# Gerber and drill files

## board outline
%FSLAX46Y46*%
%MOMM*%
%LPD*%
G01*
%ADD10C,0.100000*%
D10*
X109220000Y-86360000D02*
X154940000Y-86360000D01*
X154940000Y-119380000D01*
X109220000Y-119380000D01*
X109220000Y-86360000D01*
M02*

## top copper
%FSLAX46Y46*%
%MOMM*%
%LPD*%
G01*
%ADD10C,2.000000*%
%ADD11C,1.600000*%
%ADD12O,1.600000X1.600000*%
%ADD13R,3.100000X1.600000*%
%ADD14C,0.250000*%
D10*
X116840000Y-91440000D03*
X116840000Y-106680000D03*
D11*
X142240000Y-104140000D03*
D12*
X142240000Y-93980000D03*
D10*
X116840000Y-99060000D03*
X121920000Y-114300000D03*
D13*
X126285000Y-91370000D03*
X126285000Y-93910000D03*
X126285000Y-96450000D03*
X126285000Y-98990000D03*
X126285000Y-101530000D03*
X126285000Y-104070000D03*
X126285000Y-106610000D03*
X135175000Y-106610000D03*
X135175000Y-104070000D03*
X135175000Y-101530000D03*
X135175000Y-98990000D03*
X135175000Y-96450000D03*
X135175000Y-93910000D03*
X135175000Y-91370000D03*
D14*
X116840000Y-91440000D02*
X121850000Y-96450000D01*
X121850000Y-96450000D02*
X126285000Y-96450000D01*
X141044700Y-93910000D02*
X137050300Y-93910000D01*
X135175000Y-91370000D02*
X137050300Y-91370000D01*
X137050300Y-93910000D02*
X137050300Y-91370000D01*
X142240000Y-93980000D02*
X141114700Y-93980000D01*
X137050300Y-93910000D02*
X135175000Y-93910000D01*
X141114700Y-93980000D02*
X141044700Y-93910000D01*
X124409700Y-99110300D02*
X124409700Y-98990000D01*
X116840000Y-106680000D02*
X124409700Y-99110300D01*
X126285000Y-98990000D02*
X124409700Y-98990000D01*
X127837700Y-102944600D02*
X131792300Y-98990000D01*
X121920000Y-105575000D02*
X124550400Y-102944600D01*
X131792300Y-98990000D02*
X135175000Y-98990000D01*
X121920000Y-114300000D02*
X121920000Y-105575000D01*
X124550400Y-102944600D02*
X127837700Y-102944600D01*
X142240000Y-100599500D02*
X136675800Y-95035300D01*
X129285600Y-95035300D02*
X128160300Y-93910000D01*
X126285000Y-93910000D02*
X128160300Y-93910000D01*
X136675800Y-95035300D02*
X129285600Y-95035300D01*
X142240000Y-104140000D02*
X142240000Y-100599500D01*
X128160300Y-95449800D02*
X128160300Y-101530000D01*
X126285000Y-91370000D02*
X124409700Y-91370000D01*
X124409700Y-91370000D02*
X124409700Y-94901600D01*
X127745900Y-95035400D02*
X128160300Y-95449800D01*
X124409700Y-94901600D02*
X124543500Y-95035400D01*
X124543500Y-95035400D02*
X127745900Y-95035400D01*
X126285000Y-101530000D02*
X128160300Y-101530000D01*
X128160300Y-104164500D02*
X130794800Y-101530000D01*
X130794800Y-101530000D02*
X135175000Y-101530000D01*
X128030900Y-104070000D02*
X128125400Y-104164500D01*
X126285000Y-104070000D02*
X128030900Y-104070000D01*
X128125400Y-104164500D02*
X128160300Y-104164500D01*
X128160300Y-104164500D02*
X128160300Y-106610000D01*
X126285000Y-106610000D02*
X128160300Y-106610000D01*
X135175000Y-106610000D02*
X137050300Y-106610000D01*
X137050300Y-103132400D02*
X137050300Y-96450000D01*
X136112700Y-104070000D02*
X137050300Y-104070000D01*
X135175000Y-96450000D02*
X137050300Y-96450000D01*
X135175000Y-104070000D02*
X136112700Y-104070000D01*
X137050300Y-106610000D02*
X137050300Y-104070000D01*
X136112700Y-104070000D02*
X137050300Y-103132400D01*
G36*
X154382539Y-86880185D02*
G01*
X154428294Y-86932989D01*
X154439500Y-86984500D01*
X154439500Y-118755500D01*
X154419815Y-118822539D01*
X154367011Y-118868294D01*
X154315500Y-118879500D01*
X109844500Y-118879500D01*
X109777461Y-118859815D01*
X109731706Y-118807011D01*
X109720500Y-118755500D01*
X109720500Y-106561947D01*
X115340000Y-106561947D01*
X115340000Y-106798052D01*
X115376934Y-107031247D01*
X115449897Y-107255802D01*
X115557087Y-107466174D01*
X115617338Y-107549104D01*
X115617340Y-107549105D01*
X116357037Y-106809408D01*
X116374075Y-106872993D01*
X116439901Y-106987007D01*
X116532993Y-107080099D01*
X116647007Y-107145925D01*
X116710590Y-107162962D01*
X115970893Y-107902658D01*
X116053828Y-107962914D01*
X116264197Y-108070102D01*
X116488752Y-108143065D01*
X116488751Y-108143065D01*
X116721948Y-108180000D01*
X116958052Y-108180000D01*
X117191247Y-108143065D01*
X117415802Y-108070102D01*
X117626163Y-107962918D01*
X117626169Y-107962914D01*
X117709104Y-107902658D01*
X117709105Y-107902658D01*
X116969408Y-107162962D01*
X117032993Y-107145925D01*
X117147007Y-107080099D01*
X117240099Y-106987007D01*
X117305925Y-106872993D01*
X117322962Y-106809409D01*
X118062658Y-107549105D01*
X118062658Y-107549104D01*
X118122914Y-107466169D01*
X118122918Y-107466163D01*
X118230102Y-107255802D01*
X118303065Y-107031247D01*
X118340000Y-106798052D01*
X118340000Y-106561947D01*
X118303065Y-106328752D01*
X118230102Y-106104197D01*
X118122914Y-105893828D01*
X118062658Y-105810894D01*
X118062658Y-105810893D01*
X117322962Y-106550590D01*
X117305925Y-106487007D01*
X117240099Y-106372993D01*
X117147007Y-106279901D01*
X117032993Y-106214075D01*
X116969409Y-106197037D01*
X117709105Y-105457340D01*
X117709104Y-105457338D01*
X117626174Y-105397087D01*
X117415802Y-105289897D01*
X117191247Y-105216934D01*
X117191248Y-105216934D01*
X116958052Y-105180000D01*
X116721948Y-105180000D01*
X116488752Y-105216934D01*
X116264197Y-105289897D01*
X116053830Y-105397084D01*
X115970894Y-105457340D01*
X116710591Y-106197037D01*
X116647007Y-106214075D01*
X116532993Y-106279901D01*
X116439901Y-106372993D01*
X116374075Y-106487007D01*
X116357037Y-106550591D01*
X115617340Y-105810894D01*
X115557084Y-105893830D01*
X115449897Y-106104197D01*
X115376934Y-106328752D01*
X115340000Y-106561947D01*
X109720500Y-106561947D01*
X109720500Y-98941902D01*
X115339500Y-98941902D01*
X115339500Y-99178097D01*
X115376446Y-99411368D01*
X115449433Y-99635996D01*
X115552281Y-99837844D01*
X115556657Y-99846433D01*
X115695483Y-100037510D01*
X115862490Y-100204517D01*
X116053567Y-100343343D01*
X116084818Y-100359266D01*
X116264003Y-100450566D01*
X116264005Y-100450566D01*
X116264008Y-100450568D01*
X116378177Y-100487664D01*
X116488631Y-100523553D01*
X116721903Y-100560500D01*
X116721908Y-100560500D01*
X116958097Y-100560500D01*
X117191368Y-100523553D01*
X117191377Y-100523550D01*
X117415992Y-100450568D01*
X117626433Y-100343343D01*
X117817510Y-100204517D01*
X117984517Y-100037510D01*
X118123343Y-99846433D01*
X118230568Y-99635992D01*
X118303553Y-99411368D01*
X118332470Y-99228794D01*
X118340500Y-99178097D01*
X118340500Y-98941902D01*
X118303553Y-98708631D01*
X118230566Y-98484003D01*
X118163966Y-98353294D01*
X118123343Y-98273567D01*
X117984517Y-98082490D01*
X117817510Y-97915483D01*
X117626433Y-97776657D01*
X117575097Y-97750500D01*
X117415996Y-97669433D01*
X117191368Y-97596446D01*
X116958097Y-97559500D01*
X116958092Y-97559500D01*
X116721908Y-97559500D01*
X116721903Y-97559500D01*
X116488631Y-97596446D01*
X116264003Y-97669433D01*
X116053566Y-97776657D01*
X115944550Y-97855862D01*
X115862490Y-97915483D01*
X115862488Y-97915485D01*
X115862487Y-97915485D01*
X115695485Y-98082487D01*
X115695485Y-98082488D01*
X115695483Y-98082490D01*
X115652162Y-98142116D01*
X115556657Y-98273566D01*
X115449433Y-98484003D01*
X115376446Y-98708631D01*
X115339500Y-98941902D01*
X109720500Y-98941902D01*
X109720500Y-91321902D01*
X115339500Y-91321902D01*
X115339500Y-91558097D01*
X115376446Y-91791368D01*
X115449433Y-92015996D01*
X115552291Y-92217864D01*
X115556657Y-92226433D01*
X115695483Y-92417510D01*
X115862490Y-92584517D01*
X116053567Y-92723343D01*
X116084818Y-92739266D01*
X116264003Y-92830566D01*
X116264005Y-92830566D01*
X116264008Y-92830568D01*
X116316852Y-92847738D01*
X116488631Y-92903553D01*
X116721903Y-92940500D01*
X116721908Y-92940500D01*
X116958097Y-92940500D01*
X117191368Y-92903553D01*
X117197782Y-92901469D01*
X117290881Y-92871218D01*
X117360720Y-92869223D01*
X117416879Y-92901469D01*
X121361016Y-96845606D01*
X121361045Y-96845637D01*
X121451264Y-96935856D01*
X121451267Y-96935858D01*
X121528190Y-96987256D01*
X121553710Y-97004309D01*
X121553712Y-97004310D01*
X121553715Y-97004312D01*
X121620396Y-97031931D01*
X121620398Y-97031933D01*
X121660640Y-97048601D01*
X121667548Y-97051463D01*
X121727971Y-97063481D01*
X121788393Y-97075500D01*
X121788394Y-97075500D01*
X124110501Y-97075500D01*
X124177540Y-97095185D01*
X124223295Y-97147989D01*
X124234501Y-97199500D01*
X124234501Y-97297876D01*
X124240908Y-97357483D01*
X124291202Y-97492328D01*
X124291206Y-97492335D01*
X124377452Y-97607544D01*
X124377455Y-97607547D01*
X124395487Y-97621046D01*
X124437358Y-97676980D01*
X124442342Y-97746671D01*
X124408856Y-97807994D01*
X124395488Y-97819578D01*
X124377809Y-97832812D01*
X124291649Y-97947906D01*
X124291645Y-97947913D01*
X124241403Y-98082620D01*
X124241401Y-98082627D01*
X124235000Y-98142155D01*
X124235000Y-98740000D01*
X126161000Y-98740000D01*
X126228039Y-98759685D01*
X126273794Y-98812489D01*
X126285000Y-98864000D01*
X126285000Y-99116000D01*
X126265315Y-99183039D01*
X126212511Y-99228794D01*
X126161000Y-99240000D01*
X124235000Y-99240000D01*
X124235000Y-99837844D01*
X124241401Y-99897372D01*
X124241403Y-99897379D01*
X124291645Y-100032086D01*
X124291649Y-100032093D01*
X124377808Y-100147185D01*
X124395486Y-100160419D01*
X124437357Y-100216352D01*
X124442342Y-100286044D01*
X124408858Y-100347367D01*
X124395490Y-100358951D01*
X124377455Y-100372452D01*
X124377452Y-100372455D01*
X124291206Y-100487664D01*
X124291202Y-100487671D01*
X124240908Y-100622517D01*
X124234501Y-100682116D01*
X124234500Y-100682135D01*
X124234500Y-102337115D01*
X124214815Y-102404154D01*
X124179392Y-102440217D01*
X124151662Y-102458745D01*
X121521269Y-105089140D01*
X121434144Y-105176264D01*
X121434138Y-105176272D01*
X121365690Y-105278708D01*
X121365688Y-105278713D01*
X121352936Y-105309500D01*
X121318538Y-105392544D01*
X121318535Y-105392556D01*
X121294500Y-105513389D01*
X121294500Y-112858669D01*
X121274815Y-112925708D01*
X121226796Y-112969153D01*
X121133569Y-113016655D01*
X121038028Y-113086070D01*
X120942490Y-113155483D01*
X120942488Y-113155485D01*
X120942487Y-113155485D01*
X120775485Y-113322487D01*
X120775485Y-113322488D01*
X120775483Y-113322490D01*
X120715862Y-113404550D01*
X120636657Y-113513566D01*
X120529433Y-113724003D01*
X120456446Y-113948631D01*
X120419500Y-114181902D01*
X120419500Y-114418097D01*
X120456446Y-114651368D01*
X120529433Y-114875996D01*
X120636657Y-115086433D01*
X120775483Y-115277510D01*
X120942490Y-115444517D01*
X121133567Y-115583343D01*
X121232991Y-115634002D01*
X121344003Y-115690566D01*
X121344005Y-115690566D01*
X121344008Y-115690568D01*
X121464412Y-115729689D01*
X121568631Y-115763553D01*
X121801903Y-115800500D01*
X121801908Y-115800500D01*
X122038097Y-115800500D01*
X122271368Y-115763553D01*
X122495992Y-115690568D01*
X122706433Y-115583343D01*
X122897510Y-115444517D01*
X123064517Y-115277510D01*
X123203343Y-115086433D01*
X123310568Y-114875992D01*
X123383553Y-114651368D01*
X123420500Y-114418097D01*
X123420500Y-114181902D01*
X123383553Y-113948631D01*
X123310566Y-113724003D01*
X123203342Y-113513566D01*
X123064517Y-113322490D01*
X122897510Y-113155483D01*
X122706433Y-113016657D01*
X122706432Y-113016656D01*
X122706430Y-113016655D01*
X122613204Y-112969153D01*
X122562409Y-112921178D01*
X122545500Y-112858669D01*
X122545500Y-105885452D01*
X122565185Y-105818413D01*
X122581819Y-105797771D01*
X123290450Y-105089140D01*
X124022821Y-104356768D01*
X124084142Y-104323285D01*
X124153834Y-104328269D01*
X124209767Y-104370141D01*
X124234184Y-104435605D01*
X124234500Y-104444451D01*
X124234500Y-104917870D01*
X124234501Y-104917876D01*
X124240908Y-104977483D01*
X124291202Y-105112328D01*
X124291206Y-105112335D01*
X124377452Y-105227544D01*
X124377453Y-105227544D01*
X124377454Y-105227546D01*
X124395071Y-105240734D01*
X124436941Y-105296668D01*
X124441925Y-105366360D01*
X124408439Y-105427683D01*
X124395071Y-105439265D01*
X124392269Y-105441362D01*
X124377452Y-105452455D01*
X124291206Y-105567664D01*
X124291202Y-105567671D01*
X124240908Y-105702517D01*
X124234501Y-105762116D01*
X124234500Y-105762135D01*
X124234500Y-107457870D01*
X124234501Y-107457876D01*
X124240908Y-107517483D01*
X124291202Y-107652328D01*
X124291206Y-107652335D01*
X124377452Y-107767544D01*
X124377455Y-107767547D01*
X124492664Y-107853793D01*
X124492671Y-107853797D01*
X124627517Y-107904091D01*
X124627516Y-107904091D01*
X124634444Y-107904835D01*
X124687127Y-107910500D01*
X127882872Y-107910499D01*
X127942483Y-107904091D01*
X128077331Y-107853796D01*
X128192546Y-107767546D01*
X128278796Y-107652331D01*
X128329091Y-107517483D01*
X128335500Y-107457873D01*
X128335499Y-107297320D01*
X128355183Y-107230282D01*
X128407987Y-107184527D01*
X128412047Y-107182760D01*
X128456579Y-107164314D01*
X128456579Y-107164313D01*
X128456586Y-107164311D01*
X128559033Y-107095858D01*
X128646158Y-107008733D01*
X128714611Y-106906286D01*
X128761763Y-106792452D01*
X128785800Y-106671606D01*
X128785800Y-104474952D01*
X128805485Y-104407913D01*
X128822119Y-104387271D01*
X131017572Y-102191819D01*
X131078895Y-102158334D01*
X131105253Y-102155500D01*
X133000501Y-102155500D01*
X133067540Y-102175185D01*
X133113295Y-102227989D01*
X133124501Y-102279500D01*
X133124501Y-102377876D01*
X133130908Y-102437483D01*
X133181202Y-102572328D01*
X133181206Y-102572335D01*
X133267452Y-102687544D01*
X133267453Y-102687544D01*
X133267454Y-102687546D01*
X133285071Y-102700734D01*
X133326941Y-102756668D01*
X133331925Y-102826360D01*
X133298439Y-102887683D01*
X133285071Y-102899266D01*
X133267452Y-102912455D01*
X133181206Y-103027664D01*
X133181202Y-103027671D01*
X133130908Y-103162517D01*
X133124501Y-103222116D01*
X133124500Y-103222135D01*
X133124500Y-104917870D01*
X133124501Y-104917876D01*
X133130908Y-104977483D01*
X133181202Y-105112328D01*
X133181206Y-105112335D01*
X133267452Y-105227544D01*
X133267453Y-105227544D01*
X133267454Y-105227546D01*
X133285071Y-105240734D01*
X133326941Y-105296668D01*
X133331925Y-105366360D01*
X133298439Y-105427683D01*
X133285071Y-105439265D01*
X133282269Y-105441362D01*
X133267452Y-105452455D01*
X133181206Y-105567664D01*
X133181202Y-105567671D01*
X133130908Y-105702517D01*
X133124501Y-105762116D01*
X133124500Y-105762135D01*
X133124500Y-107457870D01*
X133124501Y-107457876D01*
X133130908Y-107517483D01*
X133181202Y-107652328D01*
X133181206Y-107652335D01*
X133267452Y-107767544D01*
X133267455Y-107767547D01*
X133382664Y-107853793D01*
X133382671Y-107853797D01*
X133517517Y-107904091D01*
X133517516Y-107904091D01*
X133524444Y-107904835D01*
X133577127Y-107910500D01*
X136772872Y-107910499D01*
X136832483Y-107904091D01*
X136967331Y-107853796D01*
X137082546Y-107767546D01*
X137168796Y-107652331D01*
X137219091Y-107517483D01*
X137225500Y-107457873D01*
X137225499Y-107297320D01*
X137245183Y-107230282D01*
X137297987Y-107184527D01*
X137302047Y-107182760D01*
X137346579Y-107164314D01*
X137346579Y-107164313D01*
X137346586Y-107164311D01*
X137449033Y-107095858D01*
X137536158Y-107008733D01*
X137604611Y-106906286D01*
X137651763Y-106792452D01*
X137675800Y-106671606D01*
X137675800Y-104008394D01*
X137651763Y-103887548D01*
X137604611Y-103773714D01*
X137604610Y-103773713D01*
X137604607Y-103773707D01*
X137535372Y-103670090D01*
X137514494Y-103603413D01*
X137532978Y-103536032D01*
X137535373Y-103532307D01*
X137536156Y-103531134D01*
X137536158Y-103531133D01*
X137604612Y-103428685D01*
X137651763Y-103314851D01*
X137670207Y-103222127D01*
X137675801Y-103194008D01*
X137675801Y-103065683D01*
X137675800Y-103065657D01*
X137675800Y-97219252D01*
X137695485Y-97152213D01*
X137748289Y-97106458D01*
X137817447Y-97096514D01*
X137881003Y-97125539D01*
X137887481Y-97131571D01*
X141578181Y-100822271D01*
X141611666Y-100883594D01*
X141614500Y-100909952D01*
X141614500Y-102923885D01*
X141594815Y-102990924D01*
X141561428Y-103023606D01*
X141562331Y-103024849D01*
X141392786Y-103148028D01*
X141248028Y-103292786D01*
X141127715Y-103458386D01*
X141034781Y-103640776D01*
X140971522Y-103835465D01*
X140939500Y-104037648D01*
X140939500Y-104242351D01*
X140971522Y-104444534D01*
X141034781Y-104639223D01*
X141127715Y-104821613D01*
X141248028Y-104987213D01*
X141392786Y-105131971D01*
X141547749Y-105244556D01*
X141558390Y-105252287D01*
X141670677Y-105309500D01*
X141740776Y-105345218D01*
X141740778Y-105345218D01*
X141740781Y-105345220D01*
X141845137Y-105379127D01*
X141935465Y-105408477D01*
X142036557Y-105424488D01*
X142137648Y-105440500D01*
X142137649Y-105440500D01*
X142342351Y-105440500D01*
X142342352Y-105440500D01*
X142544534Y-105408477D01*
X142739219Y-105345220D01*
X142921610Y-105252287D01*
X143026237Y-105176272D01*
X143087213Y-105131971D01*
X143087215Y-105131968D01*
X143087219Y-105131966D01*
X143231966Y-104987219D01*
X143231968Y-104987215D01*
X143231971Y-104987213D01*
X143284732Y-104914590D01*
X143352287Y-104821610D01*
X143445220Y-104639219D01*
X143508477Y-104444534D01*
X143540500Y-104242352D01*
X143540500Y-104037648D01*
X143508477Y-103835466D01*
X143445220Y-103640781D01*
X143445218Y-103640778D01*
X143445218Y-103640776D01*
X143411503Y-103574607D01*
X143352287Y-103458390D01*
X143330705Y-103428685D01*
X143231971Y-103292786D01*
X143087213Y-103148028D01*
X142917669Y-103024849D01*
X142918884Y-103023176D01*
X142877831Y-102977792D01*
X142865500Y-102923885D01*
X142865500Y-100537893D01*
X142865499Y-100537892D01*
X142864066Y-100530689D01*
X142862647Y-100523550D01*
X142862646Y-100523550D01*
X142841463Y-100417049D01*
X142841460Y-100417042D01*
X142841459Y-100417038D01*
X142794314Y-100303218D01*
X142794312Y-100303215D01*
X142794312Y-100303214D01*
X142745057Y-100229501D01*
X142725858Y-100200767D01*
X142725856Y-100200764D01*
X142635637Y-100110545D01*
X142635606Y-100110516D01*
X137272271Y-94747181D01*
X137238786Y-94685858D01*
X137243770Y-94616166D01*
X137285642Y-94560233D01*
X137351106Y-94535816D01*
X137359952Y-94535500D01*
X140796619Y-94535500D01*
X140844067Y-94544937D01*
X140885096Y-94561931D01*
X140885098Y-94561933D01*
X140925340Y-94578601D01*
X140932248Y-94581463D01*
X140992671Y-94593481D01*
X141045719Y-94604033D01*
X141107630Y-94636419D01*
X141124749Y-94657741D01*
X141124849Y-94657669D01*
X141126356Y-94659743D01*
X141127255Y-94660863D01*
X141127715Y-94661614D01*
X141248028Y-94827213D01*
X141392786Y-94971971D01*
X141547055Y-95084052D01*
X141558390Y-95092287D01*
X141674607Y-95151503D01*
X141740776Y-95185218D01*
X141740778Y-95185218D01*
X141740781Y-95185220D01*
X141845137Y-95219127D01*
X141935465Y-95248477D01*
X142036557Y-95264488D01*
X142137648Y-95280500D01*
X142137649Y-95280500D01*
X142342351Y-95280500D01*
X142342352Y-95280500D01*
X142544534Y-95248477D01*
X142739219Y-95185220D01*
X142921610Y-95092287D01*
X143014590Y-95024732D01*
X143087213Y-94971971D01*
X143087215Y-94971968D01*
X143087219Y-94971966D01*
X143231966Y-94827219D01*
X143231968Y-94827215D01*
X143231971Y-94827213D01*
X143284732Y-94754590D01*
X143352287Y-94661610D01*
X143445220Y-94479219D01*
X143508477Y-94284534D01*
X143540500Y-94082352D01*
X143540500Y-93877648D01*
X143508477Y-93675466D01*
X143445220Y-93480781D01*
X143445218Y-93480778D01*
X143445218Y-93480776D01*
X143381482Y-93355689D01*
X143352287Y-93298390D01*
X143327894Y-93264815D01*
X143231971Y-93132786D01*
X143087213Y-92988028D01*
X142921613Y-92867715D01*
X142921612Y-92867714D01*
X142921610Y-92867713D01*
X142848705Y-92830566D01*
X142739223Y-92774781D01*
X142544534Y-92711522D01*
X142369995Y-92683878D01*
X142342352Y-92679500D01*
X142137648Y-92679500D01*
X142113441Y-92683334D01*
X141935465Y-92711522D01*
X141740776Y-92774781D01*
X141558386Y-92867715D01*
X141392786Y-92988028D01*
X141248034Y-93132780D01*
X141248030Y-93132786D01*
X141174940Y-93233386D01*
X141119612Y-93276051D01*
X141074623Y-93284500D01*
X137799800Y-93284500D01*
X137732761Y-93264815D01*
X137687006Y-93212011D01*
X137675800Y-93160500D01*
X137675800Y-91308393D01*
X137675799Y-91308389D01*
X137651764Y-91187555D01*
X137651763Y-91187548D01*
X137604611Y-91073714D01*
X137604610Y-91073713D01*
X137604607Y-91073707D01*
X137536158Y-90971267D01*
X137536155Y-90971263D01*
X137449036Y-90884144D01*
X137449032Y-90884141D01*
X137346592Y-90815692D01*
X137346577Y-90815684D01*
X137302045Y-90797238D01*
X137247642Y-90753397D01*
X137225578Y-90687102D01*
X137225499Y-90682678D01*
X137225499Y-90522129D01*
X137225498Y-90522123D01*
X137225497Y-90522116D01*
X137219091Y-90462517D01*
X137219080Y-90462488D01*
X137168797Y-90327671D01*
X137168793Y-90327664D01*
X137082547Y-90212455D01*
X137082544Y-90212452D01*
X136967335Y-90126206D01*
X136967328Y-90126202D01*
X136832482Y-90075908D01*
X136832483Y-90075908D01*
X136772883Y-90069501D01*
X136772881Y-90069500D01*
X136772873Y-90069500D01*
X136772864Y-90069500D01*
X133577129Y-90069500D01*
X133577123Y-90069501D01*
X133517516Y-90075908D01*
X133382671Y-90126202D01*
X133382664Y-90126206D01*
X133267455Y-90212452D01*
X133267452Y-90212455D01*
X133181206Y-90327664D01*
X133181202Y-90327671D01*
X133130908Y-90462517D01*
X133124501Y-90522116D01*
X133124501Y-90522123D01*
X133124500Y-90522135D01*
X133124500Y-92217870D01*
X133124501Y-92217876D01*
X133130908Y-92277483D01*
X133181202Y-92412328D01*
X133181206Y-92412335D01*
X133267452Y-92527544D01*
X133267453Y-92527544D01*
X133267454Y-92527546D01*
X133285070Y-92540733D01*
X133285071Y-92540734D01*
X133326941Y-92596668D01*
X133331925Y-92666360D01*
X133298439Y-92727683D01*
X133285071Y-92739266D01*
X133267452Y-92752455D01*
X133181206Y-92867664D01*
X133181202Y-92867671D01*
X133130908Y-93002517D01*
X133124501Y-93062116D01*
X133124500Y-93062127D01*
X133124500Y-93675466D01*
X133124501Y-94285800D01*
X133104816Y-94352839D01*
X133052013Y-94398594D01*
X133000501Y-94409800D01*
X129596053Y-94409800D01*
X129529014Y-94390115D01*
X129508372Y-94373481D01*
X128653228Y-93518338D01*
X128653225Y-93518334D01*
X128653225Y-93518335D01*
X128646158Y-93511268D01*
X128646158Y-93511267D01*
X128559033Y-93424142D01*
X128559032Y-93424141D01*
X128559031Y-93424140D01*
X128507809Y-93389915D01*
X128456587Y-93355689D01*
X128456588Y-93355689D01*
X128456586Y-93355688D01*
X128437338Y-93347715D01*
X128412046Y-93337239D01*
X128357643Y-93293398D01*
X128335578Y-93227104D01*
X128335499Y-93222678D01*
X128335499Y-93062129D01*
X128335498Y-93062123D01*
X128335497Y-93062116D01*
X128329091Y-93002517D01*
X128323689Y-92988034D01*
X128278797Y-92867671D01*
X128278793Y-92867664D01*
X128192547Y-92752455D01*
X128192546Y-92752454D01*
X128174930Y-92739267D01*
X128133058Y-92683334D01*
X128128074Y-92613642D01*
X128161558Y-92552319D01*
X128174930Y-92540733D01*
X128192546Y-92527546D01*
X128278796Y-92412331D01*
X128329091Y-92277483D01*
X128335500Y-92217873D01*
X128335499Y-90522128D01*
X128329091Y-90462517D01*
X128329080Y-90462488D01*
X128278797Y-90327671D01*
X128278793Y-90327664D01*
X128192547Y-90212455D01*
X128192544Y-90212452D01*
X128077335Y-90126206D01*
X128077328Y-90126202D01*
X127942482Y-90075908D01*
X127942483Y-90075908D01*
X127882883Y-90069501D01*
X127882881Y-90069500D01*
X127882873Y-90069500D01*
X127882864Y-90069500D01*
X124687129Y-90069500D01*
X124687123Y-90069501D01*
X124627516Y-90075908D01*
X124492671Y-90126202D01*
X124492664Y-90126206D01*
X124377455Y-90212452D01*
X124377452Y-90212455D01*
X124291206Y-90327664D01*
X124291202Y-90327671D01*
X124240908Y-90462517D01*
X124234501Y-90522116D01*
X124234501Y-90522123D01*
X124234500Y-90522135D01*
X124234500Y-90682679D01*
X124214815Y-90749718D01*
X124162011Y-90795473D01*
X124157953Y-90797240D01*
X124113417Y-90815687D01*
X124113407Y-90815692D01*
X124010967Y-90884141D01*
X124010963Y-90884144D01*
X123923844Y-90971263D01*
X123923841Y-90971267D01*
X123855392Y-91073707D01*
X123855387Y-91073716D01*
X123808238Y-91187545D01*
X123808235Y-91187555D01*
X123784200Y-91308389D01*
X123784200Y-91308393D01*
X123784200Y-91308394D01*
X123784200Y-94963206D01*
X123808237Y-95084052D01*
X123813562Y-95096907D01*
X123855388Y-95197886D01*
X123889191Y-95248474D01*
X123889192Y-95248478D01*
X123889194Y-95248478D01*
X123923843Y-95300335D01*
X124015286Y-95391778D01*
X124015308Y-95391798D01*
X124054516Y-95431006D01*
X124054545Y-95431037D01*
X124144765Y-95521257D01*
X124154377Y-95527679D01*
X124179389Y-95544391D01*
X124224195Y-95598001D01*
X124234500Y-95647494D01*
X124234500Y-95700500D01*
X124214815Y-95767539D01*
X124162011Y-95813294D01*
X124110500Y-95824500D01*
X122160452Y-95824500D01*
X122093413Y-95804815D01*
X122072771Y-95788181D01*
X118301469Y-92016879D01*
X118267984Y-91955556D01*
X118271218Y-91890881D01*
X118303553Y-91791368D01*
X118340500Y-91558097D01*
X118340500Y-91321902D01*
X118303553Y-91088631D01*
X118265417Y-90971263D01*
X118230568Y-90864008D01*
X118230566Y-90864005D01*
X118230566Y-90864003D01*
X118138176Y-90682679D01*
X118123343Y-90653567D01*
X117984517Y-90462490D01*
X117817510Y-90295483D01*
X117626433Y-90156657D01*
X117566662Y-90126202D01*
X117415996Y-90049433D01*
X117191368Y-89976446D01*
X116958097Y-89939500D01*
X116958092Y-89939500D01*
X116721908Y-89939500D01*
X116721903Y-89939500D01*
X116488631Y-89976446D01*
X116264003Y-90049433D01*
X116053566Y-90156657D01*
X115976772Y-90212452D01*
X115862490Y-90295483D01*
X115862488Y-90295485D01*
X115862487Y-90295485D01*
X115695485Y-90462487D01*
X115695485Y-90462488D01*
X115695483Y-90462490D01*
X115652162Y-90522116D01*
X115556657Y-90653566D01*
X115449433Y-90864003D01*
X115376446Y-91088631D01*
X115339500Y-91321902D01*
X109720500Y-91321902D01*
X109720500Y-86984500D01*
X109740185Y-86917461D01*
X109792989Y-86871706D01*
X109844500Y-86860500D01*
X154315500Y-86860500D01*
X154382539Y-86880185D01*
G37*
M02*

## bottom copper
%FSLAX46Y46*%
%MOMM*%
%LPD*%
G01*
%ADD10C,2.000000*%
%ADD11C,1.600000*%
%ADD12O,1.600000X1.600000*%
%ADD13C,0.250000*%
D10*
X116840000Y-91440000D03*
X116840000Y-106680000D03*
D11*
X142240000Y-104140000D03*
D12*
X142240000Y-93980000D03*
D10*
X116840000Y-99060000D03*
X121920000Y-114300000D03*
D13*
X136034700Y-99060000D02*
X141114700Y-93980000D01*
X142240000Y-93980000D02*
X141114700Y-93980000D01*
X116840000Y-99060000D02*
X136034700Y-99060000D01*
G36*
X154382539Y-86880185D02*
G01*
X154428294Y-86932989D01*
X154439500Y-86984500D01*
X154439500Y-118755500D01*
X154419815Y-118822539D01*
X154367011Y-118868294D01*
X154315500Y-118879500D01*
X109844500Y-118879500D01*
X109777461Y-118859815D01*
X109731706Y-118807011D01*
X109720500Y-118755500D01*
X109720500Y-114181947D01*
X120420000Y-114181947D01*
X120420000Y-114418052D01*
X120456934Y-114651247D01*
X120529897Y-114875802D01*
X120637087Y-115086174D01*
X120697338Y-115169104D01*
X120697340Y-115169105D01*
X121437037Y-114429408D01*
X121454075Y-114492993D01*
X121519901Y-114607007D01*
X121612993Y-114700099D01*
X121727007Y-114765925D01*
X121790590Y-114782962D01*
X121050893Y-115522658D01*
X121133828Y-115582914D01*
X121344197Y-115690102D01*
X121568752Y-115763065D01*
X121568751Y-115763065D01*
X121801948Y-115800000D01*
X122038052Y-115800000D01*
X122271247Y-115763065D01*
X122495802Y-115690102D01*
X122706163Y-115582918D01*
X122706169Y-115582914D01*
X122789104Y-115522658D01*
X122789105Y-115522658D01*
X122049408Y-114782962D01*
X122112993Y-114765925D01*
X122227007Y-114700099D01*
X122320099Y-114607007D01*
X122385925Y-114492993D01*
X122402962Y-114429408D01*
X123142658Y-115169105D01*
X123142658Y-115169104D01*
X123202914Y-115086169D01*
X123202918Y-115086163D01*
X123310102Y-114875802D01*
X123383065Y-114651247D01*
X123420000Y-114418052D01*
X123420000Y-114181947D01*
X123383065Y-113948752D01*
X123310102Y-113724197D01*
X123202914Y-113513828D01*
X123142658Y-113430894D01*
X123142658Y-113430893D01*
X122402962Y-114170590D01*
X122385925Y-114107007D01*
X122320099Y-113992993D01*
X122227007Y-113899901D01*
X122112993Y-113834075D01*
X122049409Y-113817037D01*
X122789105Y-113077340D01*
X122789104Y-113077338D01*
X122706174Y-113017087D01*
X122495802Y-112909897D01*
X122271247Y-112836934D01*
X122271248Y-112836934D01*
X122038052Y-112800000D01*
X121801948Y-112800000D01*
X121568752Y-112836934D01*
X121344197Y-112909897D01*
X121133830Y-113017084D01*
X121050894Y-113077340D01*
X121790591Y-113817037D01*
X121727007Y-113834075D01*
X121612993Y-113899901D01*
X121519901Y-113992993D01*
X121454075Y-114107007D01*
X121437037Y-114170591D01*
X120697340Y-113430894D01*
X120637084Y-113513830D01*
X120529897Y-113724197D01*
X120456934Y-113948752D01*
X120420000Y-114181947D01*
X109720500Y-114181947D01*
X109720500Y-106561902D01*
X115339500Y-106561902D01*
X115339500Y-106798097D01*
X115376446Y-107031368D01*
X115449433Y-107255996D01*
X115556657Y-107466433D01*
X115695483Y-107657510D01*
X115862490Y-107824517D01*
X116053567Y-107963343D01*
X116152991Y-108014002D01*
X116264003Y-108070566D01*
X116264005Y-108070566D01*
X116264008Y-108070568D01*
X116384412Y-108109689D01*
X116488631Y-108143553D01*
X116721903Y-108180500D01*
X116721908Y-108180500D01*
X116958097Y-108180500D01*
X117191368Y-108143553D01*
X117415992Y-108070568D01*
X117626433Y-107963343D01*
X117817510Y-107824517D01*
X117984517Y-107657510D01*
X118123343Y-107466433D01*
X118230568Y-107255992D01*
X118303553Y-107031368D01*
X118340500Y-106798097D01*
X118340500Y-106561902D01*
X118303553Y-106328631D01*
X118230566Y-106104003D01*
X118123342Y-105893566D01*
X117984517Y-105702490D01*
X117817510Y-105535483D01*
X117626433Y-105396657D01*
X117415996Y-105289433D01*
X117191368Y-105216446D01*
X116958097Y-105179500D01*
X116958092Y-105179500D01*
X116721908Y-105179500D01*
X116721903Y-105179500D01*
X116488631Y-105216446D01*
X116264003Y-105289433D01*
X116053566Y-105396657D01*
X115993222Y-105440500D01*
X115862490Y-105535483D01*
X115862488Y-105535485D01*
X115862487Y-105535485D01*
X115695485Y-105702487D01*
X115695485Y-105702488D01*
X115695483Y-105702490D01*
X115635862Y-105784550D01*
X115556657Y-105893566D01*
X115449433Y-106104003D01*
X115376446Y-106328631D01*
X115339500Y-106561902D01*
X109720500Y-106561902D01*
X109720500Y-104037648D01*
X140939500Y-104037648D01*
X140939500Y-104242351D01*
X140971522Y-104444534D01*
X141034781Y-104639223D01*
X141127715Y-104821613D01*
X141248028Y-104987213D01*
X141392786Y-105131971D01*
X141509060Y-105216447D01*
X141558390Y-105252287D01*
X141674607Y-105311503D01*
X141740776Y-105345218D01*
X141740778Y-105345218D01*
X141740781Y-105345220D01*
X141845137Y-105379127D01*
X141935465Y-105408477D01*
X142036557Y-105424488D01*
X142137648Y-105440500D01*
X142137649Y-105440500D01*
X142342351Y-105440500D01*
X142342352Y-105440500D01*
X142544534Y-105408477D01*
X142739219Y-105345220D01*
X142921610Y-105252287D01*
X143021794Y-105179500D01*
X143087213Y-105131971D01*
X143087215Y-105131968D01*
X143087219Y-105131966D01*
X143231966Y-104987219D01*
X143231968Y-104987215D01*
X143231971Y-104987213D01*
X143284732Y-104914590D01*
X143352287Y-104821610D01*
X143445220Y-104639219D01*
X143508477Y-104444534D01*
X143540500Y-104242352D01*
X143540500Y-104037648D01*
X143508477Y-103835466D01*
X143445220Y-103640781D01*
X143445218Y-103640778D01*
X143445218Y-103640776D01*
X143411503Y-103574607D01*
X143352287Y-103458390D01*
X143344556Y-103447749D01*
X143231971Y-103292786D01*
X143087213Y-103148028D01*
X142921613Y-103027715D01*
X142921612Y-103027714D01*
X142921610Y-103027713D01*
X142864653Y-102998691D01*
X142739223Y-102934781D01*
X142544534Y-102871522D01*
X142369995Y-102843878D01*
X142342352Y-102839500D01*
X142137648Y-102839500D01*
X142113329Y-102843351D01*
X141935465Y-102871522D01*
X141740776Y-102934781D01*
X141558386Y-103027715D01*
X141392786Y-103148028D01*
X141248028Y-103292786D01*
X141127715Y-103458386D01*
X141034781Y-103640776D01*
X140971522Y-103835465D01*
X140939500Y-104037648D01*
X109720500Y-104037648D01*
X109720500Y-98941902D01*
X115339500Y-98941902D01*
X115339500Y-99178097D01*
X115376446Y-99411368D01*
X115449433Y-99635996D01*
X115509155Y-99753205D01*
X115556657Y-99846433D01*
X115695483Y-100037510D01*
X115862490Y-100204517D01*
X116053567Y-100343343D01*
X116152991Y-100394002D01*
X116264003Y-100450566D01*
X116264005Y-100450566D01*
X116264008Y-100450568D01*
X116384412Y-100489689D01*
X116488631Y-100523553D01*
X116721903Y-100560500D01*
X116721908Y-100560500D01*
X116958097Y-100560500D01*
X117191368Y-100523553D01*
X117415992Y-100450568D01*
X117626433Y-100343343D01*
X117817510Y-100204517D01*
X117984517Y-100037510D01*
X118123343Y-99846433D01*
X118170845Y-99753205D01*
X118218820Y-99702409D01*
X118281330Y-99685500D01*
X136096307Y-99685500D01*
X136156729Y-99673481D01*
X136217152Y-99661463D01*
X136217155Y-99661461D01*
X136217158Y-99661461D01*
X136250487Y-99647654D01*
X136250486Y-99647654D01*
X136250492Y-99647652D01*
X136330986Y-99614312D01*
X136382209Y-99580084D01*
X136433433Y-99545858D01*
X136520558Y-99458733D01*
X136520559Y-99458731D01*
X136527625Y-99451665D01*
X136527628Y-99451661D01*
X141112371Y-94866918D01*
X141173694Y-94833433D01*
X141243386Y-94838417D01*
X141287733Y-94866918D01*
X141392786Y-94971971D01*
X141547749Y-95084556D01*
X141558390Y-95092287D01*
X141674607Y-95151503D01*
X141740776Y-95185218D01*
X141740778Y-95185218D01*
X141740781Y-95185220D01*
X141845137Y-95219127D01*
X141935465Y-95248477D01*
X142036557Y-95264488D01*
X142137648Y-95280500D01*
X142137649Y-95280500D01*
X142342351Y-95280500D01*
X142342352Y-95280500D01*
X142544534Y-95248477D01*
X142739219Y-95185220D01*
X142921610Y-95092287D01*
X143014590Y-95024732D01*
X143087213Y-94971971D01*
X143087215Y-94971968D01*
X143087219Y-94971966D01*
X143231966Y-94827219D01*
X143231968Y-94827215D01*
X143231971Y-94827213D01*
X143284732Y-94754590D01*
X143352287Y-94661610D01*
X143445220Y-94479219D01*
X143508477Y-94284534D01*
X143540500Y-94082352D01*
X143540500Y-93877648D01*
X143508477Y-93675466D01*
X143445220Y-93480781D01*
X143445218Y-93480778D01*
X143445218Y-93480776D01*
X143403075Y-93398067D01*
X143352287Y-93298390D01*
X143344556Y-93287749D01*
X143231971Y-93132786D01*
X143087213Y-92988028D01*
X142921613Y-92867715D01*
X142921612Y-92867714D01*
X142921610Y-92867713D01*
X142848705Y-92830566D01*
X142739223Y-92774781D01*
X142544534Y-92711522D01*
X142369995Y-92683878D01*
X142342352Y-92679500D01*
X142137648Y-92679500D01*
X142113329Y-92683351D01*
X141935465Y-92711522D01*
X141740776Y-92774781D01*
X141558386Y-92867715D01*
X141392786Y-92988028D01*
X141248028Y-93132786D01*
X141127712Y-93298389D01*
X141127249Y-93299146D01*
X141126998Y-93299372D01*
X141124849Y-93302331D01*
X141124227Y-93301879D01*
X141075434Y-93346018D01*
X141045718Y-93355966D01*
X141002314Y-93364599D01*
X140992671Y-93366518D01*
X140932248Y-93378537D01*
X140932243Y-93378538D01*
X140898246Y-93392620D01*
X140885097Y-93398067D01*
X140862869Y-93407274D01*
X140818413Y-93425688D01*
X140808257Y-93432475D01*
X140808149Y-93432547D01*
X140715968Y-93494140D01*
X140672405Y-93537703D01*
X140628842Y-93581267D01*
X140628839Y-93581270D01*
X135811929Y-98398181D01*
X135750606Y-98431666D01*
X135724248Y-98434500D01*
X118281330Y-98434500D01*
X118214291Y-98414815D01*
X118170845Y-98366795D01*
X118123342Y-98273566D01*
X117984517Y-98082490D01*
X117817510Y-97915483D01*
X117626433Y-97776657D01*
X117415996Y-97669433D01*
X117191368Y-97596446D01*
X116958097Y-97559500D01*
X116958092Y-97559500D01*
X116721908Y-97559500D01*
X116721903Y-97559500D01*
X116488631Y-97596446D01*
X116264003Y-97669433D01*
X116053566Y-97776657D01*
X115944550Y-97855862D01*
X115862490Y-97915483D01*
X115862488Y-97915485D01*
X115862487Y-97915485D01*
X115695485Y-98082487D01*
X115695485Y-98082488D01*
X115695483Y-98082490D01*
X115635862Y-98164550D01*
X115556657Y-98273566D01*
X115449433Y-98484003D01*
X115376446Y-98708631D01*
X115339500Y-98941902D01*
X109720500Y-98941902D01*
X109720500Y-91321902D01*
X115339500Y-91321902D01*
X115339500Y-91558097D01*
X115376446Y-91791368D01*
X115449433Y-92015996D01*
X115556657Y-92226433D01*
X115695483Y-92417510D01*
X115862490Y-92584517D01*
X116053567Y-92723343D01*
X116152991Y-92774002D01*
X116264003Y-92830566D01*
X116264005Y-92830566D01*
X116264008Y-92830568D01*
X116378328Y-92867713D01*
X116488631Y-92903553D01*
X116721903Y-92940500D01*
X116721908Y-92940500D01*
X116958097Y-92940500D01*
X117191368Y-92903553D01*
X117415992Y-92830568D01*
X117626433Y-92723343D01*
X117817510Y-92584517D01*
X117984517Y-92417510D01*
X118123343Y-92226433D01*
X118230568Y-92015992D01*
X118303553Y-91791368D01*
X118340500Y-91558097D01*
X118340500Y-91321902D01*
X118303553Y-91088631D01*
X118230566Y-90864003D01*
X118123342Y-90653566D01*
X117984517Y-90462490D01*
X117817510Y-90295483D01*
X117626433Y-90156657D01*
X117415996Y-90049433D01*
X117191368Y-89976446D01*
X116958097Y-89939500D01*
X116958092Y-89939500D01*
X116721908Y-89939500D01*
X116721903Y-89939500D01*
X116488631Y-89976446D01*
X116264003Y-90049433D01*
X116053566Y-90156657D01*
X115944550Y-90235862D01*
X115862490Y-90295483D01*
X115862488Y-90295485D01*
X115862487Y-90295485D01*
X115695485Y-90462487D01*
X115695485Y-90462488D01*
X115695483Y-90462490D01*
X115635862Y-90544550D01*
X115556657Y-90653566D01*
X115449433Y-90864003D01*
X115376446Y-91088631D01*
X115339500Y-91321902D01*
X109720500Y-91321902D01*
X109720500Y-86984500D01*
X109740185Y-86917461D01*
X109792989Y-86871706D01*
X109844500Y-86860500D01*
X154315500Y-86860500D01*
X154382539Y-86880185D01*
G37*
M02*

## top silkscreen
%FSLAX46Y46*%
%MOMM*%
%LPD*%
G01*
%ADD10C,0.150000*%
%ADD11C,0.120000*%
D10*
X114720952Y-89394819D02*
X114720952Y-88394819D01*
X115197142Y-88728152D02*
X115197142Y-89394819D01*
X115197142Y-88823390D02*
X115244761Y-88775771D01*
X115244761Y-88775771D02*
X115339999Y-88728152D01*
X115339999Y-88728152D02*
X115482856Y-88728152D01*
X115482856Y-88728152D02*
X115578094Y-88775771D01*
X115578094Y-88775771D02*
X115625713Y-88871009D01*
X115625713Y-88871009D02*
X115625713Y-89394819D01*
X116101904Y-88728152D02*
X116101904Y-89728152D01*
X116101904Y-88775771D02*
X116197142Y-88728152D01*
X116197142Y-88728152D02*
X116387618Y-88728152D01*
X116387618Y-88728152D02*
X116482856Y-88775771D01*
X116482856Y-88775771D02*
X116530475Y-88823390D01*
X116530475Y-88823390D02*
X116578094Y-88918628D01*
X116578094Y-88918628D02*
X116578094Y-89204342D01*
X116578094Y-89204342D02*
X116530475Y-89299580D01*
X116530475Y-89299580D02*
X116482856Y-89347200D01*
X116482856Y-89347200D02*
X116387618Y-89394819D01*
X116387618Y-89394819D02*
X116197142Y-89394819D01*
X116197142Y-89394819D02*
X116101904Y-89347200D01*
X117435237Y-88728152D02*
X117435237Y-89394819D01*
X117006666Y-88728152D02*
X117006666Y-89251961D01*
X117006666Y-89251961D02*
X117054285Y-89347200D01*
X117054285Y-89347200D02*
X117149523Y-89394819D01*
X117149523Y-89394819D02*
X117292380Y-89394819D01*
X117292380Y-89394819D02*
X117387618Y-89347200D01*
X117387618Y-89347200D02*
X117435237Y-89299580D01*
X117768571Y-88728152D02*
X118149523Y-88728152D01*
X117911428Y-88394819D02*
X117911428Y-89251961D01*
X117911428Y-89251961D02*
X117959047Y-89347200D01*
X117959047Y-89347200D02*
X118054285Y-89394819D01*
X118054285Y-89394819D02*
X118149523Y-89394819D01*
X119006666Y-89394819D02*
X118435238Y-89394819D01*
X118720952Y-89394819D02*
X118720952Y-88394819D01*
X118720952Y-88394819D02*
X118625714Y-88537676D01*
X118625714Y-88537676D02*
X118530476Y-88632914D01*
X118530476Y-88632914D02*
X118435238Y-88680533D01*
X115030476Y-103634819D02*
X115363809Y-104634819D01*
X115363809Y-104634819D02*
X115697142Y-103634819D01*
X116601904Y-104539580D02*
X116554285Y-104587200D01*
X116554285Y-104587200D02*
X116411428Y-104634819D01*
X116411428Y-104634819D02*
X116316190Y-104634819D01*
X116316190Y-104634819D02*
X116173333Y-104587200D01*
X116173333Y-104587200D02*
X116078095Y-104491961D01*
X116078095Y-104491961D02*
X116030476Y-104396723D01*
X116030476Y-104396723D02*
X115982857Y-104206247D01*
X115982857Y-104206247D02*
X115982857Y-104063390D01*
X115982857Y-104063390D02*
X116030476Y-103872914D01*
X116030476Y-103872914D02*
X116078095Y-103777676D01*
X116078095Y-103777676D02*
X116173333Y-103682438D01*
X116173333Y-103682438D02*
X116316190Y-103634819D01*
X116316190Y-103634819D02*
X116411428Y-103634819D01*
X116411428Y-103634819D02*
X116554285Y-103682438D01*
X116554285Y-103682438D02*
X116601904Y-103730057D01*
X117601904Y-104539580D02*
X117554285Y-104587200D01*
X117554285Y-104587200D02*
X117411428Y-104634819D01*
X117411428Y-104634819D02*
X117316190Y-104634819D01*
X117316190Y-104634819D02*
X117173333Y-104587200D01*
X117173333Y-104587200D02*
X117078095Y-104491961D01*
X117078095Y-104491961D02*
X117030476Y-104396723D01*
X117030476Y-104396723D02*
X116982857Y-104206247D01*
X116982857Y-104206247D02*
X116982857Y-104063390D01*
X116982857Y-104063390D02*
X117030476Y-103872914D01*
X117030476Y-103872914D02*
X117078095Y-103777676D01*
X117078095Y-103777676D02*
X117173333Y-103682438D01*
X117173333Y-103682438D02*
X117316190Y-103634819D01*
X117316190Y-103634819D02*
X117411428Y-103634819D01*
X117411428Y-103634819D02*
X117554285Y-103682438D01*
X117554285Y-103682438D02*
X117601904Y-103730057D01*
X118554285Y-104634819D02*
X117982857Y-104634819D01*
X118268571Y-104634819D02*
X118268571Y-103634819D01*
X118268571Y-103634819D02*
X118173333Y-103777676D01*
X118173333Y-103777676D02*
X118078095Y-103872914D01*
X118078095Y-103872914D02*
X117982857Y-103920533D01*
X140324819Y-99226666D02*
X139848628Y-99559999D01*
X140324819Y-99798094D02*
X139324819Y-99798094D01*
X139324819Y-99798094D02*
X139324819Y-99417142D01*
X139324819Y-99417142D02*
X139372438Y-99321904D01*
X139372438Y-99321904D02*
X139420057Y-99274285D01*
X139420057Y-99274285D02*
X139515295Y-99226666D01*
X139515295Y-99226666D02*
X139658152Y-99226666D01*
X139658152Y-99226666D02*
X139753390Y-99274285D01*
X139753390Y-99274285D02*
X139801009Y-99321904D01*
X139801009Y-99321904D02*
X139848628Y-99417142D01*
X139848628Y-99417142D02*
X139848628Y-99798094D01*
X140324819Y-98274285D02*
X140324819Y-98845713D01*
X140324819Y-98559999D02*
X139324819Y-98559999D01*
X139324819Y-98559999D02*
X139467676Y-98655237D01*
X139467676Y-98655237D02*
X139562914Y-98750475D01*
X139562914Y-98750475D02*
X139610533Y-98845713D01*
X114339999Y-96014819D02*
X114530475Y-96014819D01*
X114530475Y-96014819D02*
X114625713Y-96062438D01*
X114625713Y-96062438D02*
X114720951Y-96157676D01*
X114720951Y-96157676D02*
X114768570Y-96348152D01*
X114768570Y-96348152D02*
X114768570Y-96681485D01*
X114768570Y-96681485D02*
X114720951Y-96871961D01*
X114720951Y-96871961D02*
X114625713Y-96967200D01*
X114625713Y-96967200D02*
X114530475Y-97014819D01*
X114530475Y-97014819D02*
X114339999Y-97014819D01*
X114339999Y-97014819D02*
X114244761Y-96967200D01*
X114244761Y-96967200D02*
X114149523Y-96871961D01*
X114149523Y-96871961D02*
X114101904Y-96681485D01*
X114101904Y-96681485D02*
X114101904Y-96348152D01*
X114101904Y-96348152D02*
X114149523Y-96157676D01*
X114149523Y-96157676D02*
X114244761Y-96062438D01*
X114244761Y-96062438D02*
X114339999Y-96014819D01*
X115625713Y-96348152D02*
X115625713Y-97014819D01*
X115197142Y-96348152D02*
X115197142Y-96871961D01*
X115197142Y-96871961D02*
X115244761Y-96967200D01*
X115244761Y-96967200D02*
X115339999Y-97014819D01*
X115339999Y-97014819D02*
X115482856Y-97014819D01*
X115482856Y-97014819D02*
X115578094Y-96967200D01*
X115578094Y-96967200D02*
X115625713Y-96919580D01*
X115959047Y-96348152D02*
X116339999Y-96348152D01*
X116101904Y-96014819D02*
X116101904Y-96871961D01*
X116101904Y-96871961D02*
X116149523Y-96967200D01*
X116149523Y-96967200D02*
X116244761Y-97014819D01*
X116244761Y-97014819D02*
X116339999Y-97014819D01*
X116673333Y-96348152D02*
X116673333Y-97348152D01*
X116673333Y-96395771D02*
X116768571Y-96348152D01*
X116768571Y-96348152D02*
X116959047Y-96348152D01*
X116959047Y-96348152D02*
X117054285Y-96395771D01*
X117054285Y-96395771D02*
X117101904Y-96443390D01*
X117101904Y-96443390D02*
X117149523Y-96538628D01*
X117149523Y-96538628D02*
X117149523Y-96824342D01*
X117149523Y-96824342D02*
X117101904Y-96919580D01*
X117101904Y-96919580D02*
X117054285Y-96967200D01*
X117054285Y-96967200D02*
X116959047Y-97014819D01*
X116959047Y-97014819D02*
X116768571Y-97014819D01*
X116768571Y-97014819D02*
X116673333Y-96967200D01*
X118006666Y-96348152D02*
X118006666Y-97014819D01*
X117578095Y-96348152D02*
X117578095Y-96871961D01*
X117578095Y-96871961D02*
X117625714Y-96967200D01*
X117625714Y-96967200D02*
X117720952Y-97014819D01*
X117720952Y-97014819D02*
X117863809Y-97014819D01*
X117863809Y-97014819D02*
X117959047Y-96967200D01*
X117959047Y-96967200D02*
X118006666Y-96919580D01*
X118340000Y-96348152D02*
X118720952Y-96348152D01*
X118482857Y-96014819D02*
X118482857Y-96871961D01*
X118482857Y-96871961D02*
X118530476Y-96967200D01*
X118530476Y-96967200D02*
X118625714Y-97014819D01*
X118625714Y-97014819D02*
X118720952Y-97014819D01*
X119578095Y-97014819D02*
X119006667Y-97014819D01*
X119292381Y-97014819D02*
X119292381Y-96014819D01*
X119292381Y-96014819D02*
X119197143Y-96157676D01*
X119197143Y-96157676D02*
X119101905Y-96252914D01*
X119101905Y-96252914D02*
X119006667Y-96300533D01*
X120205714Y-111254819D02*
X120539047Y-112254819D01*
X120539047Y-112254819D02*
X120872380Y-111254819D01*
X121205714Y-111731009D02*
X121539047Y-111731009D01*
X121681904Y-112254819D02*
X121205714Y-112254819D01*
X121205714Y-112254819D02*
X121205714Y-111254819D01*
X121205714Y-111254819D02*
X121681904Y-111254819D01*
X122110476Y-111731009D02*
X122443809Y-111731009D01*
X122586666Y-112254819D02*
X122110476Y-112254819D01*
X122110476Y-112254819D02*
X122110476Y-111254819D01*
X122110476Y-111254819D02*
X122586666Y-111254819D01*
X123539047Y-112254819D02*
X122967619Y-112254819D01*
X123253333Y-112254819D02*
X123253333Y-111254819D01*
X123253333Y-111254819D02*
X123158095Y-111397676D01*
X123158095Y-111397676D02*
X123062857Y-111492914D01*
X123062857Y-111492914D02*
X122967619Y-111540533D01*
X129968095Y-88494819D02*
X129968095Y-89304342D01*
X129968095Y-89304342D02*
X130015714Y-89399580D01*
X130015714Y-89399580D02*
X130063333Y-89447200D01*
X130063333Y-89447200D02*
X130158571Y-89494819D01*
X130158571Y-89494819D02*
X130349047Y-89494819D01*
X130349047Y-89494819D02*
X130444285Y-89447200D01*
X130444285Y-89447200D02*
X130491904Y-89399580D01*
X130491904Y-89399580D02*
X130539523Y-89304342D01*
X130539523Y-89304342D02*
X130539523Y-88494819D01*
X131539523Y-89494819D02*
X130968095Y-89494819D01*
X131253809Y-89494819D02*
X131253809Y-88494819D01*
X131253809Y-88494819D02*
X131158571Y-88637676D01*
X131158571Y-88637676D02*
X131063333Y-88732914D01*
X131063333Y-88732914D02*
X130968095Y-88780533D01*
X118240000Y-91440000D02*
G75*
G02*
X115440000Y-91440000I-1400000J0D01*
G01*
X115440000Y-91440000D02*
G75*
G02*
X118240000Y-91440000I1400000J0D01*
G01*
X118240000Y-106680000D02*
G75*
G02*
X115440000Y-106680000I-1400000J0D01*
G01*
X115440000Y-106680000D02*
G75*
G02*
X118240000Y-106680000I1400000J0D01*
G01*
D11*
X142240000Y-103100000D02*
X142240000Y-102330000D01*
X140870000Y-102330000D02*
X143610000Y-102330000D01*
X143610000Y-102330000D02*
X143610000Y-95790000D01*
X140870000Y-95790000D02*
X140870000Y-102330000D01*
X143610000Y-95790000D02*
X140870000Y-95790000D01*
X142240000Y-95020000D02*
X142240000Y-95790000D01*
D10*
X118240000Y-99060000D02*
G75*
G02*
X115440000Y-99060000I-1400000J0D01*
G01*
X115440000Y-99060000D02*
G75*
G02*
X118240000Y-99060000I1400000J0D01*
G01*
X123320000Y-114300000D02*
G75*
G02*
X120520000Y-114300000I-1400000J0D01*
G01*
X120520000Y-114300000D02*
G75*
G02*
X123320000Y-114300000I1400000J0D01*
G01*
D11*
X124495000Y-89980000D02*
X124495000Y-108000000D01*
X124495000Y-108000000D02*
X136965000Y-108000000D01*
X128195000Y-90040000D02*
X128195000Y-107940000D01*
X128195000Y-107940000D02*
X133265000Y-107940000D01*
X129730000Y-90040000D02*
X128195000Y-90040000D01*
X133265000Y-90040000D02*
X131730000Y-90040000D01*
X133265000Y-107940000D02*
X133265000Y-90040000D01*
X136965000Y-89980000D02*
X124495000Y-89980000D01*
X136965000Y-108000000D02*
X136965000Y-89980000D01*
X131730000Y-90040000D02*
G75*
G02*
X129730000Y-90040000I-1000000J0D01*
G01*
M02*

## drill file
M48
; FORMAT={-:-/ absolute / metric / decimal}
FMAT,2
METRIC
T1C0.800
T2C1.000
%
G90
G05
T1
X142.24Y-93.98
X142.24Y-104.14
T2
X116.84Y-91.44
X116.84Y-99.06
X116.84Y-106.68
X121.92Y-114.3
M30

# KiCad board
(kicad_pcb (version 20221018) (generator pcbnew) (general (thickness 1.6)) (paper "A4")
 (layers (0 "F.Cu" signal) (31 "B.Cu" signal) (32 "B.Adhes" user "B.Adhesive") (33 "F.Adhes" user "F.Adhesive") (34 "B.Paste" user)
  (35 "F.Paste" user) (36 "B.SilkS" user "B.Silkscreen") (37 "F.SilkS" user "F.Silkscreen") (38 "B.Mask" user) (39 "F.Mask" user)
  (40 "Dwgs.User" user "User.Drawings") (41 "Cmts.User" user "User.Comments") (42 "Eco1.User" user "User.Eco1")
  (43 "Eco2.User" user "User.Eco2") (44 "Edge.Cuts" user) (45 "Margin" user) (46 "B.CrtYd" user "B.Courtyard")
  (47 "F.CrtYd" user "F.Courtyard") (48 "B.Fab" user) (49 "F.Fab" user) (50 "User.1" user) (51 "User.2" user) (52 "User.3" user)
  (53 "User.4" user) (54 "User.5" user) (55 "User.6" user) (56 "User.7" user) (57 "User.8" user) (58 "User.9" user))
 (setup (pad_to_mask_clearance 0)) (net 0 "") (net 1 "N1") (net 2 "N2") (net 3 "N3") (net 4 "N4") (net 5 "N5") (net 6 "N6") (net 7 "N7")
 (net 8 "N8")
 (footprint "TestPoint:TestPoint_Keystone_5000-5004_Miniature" (layer "F.Cu") (at 116.84 91.44)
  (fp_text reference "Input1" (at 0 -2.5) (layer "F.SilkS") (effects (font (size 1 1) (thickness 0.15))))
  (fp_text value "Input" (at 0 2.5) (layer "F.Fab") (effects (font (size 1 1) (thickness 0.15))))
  (fp_circle (center 0 0) (end 1.4 0) (stroke (width 0.15) (type solid)) (fill none) (layer "F.SilkS"))
  (pad "1" thru_hole circle (at 0 0) (size 2 2) (drill 1) (layers "*.Cu" "*.Mask") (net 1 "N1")))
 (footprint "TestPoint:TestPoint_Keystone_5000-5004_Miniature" (layer "F.Cu") (at 116.84 106.68)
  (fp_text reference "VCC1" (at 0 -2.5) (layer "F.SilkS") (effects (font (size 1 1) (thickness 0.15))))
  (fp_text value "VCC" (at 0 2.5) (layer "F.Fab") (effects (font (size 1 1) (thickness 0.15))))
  (fp_circle (center 0 0) (end 1.4 0) (stroke (width 0.15) (type solid)) (fill none) (layer "F.SilkS"))
  (pad "1" thru_hole circle (at 0 0) (size 2 2) (drill 1) (layers "*.Cu" "*.Mask") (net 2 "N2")))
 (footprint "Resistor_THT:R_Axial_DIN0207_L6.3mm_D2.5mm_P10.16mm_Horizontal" (layer "F.Cu") (at 142.24 104.14 90)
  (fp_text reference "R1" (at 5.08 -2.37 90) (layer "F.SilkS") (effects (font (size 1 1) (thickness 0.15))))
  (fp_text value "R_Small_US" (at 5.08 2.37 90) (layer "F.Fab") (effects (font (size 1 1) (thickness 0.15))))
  (fp_line (start 1.04 0) (end 1.81 0) (stroke (width 0.12) (type solid)) (layer "F.SilkS"))
  (fp_line (start 1.81 -1.37) (end 1.81 1.37) (stroke (width 0.12) (type solid)) (layer "F.SilkS"))
  (fp_line (start 1.81 1.37) (end 8.35 1.37) (stroke (width 0.12) (type solid)) (layer "F.SilkS"))
  (fp_line (start 8.35 -1.37) (end 1.81 -1.37) (stroke (width 0.12) (type solid)) (layer "F.SilkS"))
  (fp_line (start 8.35 1.37) (end 8.35 -1.37) (stroke (width 0.12) (type solid)) (layer "F.SilkS"))
  (fp_line (start 9.12 0) (end 8.35 0) (stroke (width 0.12) (type solid)) (layer "F.SilkS"))
  (pad "1" thru_hole circle (at 0 0 90) (size 1.6 1.6) (drill 0.8) (layers "*.Cu" "*.Mask") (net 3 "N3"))
  (pad "2" thru_hole oval (at 10.16 0 90) (size 1.6 1.6) (drill 0.8) (layers "*.Cu" "*.Mask") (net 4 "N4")))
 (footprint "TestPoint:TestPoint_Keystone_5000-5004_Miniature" (layer "F.Cu") (at 116.84 99.06)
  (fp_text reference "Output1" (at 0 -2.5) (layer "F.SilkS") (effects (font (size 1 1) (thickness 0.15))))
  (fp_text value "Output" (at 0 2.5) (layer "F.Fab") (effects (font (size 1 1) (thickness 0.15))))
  (fp_circle (center 0 0) (end 1.4 0) (stroke (width 0.15) (type solid)) (fill none) (layer "F.SilkS"))
  (pad "1" thru_hole circle (at 0 0) (size 2 2) (drill 1) (layers "*.Cu" "*.Mask") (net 4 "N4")))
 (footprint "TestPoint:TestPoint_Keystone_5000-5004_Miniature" (layer "F.Cu") (at 121.92 114.3)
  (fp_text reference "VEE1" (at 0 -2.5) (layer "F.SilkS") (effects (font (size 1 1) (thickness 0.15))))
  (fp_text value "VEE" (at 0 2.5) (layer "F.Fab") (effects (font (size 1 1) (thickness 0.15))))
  (fp_circle (center 0 0) (end 1.4 0) (stroke (width 0.15) (type solid)) (fill none) (layer "F.SilkS"))
  (pad "1" thru_hole circle (at 0 0) (size 2 2) (drill 1) (layers "*.Cu" "*.Mask") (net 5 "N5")))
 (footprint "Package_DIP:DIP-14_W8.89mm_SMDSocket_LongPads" (layer "F.Cu") (at 130.73 98.99)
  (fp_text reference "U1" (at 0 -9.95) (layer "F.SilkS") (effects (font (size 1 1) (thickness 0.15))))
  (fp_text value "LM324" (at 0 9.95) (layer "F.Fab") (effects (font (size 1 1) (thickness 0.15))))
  (fp_line (start -6.235 -9.01) (end -6.235 9.01) (stroke (width 0.12) (type solid)) (layer "F.SilkS"))
  (fp_line (start -6.235 9.01) (end 6.235 9.01) (stroke (width 0.12) (type solid)) (layer "F.SilkS"))
  (fp_line (start -2.535 -8.95) (end -2.535 8.95) (stroke (width 0.12) (type solid)) (layer "F.SilkS"))
  (fp_line (start -2.535 8.95) (end 2.535 8.95) (stroke (width 0.12) (type solid)) (layer "F.SilkS"))
  (fp_line (start -1 -8.95) (end -2.535 -8.95) (stroke (width 0.12) (type solid)) (layer "F.SilkS"))
  (fp_line (start 2.535 -8.95) (end 1 -8.95) (stroke (width 0.12) (type solid)) (layer "F.SilkS"))
  (fp_line (start 2.535 8.95) (end 2.535 -8.95) (stroke (width 0.12) (type solid)) (layer "F.SilkS"))
  (fp_line (start 6.235 -9.01) (end -6.235 -9.01) (stroke (width 0.12) (type solid)) (layer "F.SilkS"))
  (fp_line (start 6.235 9.01) (end 6.235 -9.01) (stroke (width 0.12) (type solid)) (layer "F.SilkS"))
  (fp_arc (start 1 -8.95) (mid 0 -7.95) (end -1 -8.95) (stroke (width 0.12) (type solid)) (layer "F.SilkS"))
  (pad "1" smd rect (at -4.445 -7.62) (size 3.1 1.6) (layers "F.Cu" "F.Paste" "F.Mask") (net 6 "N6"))
  (pad "2" smd rect (at -4.445 -5.08) (size 3.1 1.6) (layers "F.Cu" "F.Paste" "F.Mask") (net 3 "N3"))
  (pad "3" smd rect (at -4.445 -2.54) (size 3.1 1.6) (layers "F.Cu" "F.Paste" "F.Mask") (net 1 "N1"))
  (pad "4" smd rect (at -4.445 0) (size 3.1 1.6) (layers "F.Cu" "F.Paste" "F.Mask") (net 2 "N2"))
  (pad "5" smd rect (at -4.445 2.54) (size 3.1 1.6) (layers "F.Cu" "F.Paste" "F.Mask") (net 6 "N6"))
  (pad "6" smd rect (at -4.445 5.08) (size 3.1 1.6) (layers "F.Cu" "F.Paste" "F.Mask") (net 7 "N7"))
  (pad "7" smd rect (at -4.445 7.62) (size 3.1 1.6) (layers "F.Cu" "F.Paste" "F.Mask") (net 7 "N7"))
  (pad "8" smd rect (at 4.445 7.62) (size 3.1 1.6) (layers "F.Cu" "F.Paste" "F.Mask") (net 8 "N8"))
  (pad "9" smd rect (at 4.445 5.08) (size 3.1 1.6) (layers "F.Cu" "F.Paste" "F.Mask") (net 8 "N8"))
  (pad "10" smd rect (at 4.445 2.54) (size 3.1 1.6) (layers "F.Cu" "F.Paste" "F.Mask") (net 7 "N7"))
  (pad "11" smd rect (at 4.445 0) (size 3.1 1.6) (layers "F.Cu" "F.Paste" "F.Mask") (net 5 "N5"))
  (pad "12" smd rect (at 4.445 -2.54) (size 3.1 1.6) (layers "F.Cu" "F.Paste" "F.Mask") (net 8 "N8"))
  (pad "13" smd rect (at 4.445 -5.08) (size 3.1 1.6) (layers "F.Cu" "F.Paste" "F.Mask") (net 4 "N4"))
  (pad "14" smd rect (at 4.445 -7.62) (size 3.1 1.6) (layers "F.Cu" "F.Paste" "F.Mask") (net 4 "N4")))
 (gr_rect (start 109.22 86.36) (end 154.94 119.38) (stroke (width 0.1) (type default)) (fill none) (layer "Edge.Cuts"))
 (segment (start 116.84 91.44) (end 121.85 96.45) (width 0.25) (layer "F.Cu") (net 1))
 (segment (start 121.85 96.45) (end 126.285 96.45) (width 0.25) (layer "F.Cu") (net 1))
 (segment (start 141.0447 93.91) (end 137.0503 93.91) (width 0.25) (layer "F.Cu") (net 4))
 (segment (start 135.175 91.37) (end 137.0503 91.37) (width 0.25) (layer "F.Cu") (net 4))
 (segment (start 137.0503 93.91) (end 137.0503 91.37) (width 0.25) (layer "F.Cu") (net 4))
 (segment (start 142.24 93.98) (end 141.1147 93.98) (width 0.25) (layer "F.Cu") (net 4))
 (segment (start 137.0503 93.91) (end 135.175 93.91) (width 0.25) (layer "F.Cu") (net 4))
 (segment (start 141.1147 93.98) (end 141.0447 93.91) (width 0.25) (layer "F.Cu") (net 4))
 (segment (start 136.0347 99.06) (end 141.1147 93.98) (width 0.25) (layer "B.Cu") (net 4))
 (segment (start 142.24 93.98) (end 141.1147 93.98) (width 0.25) (layer "B.Cu") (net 4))
 (segment (start 116.84 99.06) (end 136.0347 99.06) (width 0.25) (layer "B.Cu") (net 4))
 (segment (start 124.4097 99.1103) (end 124.4097 98.99) (width 0.25) (layer "F.Cu") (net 2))
 (segment (start 116.84 106.68) (end 124.4097 99.1103) (width 0.25) (layer "F.Cu") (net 2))
 (segment (start 126.285 98.99) (end 124.4097 98.99) (width 0.25) (layer "F.Cu") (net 2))
 (segment (start 127.8377 102.9446) (end 131.7923 98.99) (width 0.25) (layer "F.Cu") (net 5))
 (segment (start 121.92 105.575) (end 124.5504 102.9446) (width 0.25) (layer "F.Cu") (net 5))
 (segment (start 131.7923 98.99) (end 135.175 98.99) (width 0.25) (layer "F.Cu") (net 5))
 (segment (start 121.92 114.3) (end 121.92 105.575) (width 0.25) (layer "F.Cu") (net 5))
 (segment (start 124.5504 102.9446) (end 127.8377 102.9446) (width 0.25) (layer "F.Cu") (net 5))
 (segment (start 142.24 100.5995) (end 136.6758 95.0353) (width 0.25) (layer "F.Cu") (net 3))
 (segment (start 129.2856 95.0353) (end 128.1603 93.91) (width 0.25) (layer "F.Cu") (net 3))
 (segment (start 126.285 93.91) (end 128.1603 93.91) (width 0.25) (layer "F.Cu") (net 3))
 (segment (start 136.6758 95.0353) (end 129.2856 95.0353) (width 0.25) (layer "F.Cu") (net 3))
 (segment (start 142.24 104.14) (end 142.24 100.5995) (width 0.25) (layer "F.Cu") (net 3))
 (segment (start 128.1603 95.4498) (end 128.1603 101.53) (width 0.25) (layer "F.Cu") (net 6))
 (segment (start 126.285 91.37) (end 124.4097 91.37) (width 0.25) (layer "F.Cu") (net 6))
 (segment (start 124.4097 91.37) (end 124.4097 94.9016) (width 0.25) (layer "F.Cu") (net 6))
 (segment (start 127.7459 95.0354) (end 128.1603 95.4498) (width 0.25) (layer "F.Cu") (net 6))
 (segment (start 124.4097 94.9016) (end 124.5435 95.0354) (width 0.25) (layer "F.Cu") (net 6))
 (segment (start 124.5435 95.0354) (end 127.7459 95.0354) (width 0.25) (layer "F.Cu") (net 6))
 (segment (start 126.285 101.53) (end 128.1603 101.53) (width 0.25) (layer "F.Cu") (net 6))
 (segment (start 128.1603 104.1645) (end 130.7948 101.53) (width 0.25) (layer "F.Cu") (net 7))
 (segment (start 130.7948 101.53) (end 135.175 101.53) (width 0.25) (layer "F.Cu") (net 7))
 (segment (start 128.0309 104.07) (end 128.1254 104.1645) (width 0.25) (layer "F.Cu") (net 7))
 (segment (start 126.285 104.07) (end 128.0309 104.07) (width 0.25) (layer "F.Cu") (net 7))
 (segment (start 128.1254 104.1645) (end 128.1603 104.1645) (width 0.25) (layer "F.Cu") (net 7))
 (segment (start 128.1603 104.1645) (end 128.1603 106.61) (width 0.25) (layer "F.Cu") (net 7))
 (segment (start 126.285 106.61) (end 128.1603 106.61) (width 0.25) (layer "F.Cu") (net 7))
 (segment (start 135.175 106.61) (end 137.0503 106.61) (width 0.25) (layer "F.Cu") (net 8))
 (segment (start 137.0503 103.1324) (end 137.0503 96.45) (width 0.25) (layer "F.Cu") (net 8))
 (segment (start 136.1127 104.07) (end 137.0503 104.07) (width 0.25) (layer "F.Cu") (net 8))
 (segment (start 135.175 96.45) (end 137.0503 96.45) (width 0.25) (layer "F.Cu") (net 8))
 (segment (start 135.175 104.07) (end 136.1127 104.07) (width 0.25) (layer "F.Cu") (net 8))
 (segment (start 137.0503 106.61) (end 137.0503 104.07) (width 0.25) (layer "F.Cu") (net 8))
 (segment (start 136.1127 104.07) (end 137.0503 103.1324) (width 0.25) (layer "F.Cu") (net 8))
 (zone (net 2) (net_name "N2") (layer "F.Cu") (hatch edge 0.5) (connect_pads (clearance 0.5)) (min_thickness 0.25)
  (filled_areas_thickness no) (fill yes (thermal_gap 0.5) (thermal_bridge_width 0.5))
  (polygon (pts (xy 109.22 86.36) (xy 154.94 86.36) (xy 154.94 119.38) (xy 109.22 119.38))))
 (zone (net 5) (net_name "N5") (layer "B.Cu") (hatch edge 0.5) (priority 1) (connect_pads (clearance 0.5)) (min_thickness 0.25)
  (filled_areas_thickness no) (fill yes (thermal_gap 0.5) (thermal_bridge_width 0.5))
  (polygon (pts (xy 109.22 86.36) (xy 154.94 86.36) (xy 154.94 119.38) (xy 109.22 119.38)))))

